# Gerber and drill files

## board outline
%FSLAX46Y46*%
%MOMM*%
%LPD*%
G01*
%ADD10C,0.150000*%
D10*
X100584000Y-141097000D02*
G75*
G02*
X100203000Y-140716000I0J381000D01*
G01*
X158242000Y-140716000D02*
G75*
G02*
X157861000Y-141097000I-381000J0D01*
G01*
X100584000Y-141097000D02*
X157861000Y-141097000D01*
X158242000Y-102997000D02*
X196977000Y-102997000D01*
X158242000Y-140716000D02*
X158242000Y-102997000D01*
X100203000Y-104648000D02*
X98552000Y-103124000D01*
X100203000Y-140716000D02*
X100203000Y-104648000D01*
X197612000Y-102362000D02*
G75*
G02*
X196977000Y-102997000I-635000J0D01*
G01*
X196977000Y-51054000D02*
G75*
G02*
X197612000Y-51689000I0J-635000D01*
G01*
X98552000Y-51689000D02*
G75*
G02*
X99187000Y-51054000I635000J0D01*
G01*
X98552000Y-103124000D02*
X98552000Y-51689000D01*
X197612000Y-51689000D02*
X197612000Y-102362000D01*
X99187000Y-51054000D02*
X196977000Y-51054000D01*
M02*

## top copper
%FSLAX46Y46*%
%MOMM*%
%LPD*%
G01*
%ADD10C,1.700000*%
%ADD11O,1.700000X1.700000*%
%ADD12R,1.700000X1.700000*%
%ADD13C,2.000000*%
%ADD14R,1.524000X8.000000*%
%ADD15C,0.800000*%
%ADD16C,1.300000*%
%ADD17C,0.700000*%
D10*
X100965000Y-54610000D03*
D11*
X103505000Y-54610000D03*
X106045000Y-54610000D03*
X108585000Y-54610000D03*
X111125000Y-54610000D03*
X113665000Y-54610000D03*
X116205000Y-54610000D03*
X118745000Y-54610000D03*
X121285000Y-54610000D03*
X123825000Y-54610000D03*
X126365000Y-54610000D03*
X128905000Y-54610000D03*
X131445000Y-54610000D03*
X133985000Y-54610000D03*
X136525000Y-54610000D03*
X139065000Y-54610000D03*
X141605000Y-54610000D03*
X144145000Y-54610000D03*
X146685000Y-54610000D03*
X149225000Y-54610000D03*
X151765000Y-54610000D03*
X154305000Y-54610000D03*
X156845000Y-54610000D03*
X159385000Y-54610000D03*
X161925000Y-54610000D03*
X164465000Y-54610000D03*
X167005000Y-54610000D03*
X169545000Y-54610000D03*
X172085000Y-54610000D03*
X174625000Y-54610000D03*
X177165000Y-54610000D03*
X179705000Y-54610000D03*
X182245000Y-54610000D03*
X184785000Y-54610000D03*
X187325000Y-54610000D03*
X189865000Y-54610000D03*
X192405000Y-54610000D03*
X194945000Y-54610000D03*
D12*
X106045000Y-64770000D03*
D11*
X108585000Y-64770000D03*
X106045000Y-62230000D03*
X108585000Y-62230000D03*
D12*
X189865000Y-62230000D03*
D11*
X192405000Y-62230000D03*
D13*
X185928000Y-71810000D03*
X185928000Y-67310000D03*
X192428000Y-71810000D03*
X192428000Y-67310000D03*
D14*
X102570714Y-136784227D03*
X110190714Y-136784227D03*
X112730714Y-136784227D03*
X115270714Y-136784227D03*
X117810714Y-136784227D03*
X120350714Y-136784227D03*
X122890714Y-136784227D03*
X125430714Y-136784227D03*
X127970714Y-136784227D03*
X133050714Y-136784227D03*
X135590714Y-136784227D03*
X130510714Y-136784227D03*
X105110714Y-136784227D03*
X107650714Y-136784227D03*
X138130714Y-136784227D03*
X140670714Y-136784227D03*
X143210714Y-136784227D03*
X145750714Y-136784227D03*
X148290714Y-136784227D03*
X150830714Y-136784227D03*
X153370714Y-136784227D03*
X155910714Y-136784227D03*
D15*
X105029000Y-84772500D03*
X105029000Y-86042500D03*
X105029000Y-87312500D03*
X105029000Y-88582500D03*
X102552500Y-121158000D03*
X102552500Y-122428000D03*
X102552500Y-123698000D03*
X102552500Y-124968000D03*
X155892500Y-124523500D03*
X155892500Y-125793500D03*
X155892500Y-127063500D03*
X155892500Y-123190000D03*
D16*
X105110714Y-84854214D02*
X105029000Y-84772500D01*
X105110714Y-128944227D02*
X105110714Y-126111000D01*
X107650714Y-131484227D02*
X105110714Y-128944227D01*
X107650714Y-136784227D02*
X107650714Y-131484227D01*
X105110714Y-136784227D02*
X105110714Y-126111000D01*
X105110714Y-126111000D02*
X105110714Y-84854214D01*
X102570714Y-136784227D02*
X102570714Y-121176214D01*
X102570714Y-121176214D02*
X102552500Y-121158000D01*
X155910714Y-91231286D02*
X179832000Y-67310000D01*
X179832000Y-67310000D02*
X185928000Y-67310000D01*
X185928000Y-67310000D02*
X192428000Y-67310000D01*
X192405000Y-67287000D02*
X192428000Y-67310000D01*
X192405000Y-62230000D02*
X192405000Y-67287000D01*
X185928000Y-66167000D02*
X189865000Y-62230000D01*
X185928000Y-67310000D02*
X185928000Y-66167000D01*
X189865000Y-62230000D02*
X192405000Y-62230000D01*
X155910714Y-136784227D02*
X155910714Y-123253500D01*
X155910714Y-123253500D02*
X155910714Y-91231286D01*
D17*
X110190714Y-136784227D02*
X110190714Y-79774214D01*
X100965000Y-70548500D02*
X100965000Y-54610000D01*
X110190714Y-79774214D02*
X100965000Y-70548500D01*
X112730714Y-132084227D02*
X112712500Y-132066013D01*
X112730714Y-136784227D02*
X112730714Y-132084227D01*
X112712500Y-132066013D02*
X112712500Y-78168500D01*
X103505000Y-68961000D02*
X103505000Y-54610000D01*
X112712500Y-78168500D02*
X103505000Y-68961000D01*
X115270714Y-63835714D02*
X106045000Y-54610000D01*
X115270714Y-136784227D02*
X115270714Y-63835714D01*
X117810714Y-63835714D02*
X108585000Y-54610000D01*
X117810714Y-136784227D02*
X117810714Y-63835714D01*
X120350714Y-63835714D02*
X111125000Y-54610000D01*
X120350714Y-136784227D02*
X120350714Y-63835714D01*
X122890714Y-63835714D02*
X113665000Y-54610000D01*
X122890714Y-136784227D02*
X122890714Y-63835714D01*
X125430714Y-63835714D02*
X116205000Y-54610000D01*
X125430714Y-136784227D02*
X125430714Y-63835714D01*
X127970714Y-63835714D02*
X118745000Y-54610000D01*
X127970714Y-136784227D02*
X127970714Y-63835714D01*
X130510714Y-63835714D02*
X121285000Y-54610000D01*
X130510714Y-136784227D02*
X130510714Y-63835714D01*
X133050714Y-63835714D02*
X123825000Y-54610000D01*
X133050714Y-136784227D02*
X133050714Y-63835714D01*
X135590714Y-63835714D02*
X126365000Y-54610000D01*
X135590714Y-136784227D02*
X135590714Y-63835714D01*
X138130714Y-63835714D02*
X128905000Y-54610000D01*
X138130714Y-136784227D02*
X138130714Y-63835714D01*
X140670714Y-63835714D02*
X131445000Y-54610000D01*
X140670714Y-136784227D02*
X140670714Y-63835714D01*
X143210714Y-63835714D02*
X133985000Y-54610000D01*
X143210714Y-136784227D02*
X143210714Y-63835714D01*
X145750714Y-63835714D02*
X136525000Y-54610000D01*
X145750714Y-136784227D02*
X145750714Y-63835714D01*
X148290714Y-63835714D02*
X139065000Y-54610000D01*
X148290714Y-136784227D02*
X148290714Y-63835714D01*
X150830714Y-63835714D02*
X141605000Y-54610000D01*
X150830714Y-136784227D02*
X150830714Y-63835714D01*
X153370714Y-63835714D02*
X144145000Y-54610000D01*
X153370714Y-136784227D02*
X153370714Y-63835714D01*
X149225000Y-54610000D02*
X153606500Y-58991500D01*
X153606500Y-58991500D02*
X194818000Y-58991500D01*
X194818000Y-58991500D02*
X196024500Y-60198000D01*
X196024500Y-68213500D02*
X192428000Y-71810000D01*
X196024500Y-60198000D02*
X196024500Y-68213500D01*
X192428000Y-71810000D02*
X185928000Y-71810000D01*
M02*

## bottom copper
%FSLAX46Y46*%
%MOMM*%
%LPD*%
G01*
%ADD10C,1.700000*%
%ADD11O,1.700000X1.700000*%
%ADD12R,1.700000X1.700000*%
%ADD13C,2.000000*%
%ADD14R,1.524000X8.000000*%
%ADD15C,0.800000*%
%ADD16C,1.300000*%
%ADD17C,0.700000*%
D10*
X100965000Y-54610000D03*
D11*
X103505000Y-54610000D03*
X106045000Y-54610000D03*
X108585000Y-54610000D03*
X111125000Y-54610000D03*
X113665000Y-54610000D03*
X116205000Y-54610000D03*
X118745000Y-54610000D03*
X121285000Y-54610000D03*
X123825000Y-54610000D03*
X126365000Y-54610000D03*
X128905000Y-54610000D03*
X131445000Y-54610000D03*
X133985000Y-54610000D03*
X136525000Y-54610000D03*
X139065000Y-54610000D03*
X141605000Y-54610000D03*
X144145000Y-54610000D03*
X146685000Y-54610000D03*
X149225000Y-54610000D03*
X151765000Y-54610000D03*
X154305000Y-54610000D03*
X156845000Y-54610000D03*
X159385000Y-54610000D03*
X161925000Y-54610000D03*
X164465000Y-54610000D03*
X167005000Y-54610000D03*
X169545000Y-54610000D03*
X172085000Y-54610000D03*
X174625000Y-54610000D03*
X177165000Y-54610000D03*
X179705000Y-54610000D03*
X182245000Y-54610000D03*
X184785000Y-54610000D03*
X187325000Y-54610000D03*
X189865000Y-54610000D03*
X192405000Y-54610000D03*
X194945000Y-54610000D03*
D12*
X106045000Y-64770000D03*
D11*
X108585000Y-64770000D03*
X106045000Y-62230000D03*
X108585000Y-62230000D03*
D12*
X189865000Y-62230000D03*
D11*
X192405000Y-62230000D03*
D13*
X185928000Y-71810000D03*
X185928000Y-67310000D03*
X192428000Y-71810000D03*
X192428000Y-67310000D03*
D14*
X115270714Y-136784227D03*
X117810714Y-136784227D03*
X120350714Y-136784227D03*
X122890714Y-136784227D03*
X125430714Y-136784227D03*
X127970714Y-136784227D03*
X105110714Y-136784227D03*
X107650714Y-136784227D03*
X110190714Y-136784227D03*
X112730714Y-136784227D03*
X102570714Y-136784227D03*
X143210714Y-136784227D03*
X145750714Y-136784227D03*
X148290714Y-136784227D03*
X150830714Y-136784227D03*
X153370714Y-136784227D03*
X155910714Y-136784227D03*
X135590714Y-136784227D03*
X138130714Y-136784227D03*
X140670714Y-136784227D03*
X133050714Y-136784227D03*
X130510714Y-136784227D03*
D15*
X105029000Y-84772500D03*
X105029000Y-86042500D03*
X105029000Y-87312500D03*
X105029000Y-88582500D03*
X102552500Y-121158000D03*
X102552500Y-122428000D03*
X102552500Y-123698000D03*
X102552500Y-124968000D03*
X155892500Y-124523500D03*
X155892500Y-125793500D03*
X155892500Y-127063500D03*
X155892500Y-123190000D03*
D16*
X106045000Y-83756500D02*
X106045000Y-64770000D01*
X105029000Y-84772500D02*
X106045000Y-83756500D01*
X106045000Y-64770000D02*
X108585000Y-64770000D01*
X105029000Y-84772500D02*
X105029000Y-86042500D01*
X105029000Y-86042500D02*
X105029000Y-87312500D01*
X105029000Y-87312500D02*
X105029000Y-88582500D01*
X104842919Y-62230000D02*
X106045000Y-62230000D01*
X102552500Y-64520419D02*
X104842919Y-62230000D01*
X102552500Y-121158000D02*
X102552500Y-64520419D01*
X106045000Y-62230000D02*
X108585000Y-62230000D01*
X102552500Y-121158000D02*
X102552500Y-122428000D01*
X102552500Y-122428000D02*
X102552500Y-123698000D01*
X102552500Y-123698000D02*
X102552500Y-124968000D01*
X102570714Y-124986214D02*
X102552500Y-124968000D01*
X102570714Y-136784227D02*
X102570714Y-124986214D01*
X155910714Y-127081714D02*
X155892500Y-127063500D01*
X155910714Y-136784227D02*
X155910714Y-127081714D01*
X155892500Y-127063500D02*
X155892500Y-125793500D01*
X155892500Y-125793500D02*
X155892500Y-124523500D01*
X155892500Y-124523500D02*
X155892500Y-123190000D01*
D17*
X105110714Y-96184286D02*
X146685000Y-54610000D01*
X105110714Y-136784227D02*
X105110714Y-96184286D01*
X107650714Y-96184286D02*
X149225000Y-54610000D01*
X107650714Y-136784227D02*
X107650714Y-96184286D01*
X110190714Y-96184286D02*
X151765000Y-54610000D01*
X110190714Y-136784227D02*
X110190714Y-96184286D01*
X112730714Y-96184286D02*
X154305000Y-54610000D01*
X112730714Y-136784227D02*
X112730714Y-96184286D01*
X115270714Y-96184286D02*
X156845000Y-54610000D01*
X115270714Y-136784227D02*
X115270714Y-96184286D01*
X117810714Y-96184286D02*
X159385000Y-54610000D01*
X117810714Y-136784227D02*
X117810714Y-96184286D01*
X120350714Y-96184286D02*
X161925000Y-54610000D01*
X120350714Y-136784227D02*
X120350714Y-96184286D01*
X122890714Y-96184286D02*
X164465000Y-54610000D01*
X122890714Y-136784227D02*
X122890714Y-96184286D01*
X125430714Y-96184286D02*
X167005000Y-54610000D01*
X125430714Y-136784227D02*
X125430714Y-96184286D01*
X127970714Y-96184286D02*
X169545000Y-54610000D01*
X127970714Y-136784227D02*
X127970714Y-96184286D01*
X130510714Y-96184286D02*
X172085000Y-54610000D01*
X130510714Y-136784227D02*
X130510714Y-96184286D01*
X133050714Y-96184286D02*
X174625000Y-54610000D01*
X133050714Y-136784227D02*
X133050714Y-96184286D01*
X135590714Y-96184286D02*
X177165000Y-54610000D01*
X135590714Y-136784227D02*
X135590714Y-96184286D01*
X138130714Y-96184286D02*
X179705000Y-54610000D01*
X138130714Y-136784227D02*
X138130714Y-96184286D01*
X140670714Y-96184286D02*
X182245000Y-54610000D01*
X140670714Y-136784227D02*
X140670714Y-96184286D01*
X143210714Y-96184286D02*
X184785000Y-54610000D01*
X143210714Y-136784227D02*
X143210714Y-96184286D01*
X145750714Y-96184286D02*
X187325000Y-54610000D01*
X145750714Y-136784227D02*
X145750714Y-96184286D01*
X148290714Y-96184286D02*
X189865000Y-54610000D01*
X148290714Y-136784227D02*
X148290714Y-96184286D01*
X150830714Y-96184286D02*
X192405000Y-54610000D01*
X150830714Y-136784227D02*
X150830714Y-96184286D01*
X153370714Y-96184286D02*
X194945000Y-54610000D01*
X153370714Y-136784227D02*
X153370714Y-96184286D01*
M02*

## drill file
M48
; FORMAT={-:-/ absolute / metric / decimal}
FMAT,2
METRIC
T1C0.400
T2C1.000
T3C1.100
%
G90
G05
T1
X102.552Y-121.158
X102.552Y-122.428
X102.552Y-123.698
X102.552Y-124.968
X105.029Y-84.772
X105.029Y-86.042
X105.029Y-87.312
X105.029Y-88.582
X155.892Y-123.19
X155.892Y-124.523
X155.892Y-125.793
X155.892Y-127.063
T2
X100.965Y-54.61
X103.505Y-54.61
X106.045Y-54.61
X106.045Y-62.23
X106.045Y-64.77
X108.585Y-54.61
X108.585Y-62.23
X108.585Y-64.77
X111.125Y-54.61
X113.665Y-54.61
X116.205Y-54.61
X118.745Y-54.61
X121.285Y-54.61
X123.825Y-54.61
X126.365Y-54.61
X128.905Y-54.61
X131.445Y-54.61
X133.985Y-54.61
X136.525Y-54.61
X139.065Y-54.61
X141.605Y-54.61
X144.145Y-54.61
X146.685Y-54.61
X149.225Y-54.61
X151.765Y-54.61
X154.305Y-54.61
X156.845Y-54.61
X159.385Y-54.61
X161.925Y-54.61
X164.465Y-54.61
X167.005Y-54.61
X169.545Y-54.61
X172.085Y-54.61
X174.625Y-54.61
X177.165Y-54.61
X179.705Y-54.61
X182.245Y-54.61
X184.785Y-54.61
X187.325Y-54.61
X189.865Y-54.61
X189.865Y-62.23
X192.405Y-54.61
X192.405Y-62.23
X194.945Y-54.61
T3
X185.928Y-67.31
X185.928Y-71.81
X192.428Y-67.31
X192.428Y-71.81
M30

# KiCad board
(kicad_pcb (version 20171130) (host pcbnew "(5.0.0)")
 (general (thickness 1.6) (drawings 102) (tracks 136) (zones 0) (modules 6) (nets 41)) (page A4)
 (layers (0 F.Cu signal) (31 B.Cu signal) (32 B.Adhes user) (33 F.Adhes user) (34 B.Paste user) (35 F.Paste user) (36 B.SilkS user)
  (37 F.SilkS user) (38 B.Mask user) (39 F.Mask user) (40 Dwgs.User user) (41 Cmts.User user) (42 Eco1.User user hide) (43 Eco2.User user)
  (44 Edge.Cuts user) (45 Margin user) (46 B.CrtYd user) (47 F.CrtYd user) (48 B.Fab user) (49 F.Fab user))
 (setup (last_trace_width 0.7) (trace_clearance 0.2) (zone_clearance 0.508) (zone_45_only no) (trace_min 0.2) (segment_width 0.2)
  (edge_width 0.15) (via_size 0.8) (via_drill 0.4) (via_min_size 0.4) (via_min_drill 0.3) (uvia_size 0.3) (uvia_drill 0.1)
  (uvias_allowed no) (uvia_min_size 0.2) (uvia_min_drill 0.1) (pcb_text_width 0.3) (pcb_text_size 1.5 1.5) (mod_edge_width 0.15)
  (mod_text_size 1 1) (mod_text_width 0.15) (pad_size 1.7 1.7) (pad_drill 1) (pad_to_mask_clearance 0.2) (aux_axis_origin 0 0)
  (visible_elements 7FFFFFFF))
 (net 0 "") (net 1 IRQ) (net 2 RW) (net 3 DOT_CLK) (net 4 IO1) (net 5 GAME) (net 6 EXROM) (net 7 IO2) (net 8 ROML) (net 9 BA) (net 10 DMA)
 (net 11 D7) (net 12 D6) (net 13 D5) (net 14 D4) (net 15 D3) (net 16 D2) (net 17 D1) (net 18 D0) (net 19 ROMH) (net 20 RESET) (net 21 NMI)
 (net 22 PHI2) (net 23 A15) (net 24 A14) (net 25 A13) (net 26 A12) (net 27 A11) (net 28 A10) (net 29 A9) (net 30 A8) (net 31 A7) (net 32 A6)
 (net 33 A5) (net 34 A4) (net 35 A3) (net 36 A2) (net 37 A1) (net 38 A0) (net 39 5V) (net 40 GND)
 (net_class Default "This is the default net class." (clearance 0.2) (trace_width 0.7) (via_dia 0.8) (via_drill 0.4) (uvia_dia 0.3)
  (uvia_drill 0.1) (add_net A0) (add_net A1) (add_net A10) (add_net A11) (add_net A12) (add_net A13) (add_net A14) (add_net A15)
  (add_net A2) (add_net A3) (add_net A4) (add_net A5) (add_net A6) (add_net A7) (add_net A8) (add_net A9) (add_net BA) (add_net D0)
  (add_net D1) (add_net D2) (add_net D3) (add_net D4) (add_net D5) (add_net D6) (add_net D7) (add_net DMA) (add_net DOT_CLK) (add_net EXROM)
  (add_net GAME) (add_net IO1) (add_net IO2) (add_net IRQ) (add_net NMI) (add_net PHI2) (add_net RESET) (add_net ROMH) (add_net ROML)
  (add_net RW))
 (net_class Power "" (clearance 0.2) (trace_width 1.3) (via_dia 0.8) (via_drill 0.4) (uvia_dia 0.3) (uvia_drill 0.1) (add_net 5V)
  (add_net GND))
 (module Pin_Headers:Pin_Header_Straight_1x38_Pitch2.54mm (layer B.Cu) (at 100.965 54.61 270)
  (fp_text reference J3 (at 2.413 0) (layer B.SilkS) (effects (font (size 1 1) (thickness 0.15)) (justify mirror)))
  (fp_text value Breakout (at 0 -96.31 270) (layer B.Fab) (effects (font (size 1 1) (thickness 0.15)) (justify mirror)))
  (pad 1 thru_hole circle (at 0 0 270) (size 1.7 1.7) (drill 1) (layers *.Cu *.Mask) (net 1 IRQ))
  (pad 2 thru_hole oval (at 0 -2.54 270) (size 1.7 1.7) (drill 1) (layers *.Cu *.Mask) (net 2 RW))
  (pad 3 thru_hole oval (at 0 -5.08 270) (size 1.7 1.7) (drill 1) (layers *.Cu *.Mask) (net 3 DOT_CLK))
  (pad 4 thru_hole oval (at 0 -7.62 270) (size 1.7 1.7) (drill 1) (layers *.Cu *.Mask) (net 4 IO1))
  (pad 5 thru_hole oval (at 0 -10.16 270) (size 1.7 1.7) (drill 1) (layers *.Cu *.Mask) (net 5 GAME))
  (pad 6 thru_hole oval (at 0 -12.7 270) (size 1.7 1.7) (drill 1) (layers *.Cu *.Mask) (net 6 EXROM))
  (pad 7 thru_hole oval (at 0 -15.24 270) (size 1.7 1.7) (drill 1) (layers *.Cu *.Mask) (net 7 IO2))
  (pad 8 thru_hole oval (at 0 -17.78 270) (size 1.7 1.7) (drill 1) (layers *.Cu *.Mask) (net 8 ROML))
  (pad 9 thru_hole oval (at 0 -20.32 270) (size 1.7 1.7) (drill 1) (layers *.Cu *.Mask) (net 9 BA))
  (pad 10 thru_hole oval (at 0 -22.86 270) (size 1.7 1.7) (drill 1) (layers *.Cu *.Mask) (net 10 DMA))
  (pad 11 thru_hole oval (at 0 -25.4 270) (size 1.7 1.7) (drill 1) (layers *.Cu *.Mask) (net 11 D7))
  (pad 12 thru_hole oval (at 0 -27.94 270) (size 1.7 1.7) (drill 1) (layers *.Cu *.Mask) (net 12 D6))
  (pad 13 thru_hole oval (at 0 -30.48 270) (size 1.7 1.7) (drill 1) (layers *.Cu *.Mask) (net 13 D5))
  (pad 14 thru_hole oval (at 0 -33.02 270) (size 1.7 1.7) (drill 1) (layers *.Cu *.Mask) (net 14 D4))
  (pad 15 thru_hole oval (at 0 -35.56 270) (size 1.7 1.7) (drill 1) (layers *.Cu *.Mask) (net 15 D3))
  (pad 16 thru_hole oval (at 0 -38.1 270) (size 1.7 1.7) (drill 1) (layers *.Cu *.Mask) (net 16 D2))
  (pad 17 thru_hole oval (at 0 -40.64 270) (size 1.7 1.7) (drill 1) (layers *.Cu *.Mask) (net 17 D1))
  (pad 18 thru_hole oval (at 0 -43.18 270) (size 1.7 1.7) (drill 1) (layers *.Cu *.Mask) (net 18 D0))
  (pad 19 thru_hole oval (at 0 -45.72 270) (size 1.7 1.7) (drill 1) (layers *.Cu *.Mask) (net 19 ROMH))
  (pad 20 thru_hole oval (at 0 -48.26 270) (size 1.7 1.7) (drill 1) (layers *.Cu *.Mask) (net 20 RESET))
  (pad 21 thru_hole oval (at 0 -50.8 270) (size 1.7 1.7) (drill 1) (layers *.Cu *.Mask) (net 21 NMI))
  (pad 22 thru_hole oval (at 0 -53.34 270) (size 1.7 1.7) (drill 1) (layers *.Cu *.Mask) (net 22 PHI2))
  (pad 23 thru_hole oval (at 0 -55.88 270) (size 1.7 1.7) (drill 1) (layers *.Cu *.Mask) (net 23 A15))
  (pad 24 thru_hole oval (at 0 -58.42 270) (size 1.7 1.7) (drill 1) (layers *.Cu *.Mask) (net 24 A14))
  (pad 25 thru_hole oval (at 0 -60.96 270) (size 1.7 1.7) (drill 1) (layers *.Cu *.Mask) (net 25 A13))
  (pad 26 thru_hole oval (at 0 -63.5 270) (size 1.7 1.7) (drill 1) (layers *.Cu *.Mask) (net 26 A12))
  (pad 27 thru_hole oval (at 0 -66.04 270) (size 1.7 1.7) (drill 1) (layers *.Cu *.Mask) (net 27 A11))
  (pad 28 thru_hole oval (at 0 -68.58 270) (size 1.7 1.7) (drill 1) (layers *.Cu *.Mask) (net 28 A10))
  (pad 29 thru_hole oval (at 0 -71.12 270) (size 1.7 1.7) (drill 1) (layers *.Cu *.Mask) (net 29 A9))
  (pad 30 thru_hole oval (at 0 -73.66 270) (size 1.7 1.7) (drill 1) (layers *.Cu *.Mask) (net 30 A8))
  (pad 31 thru_hole oval (at 0 -76.2 270) (size 1.7 1.7) (drill 1) (layers *.Cu *.Mask) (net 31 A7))
  (pad 32 thru_hole oval (at 0 -78.74 270) (size 1.7 1.7) (drill 1) (layers *.Cu *.Mask) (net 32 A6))
  (pad 33 thru_hole oval (at 0 -81.28 270) (size 1.7 1.7) (drill 1) (layers *.Cu *.Mask) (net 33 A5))
  (pad 34 thru_hole oval (at 0 -83.82 270) (size 1.7 1.7) (drill 1) (layers *.Cu *.Mask) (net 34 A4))
  (pad 35 thru_hole oval (at 0 -86.36 270) (size 1.7 1.7) (drill 1) (layers *.Cu *.Mask) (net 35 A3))
  (pad 36 thru_hole oval (at 0 -88.9 270) (size 1.7 1.7) (drill 1) (layers *.Cu *.Mask) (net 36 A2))
  (pad 37 thru_hole oval (at 0 -91.44 270) (size 1.7 1.7) (drill 1) (layers *.Cu *.Mask) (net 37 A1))
  (pad 38 thru_hole oval (at 0 -93.98 270) (size 1.7 1.7) (drill 1) (layers *.Cu *.Mask) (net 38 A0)))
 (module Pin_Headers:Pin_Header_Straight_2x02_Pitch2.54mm (layer B.Cu) (at 106.045 64.77)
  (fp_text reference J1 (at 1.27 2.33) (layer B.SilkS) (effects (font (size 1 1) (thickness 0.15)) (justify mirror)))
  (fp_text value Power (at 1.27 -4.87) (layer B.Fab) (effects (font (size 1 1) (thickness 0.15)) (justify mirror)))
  (pad 1 thru_hole rect (at 0 0) (size 1.7 1.7) (drill 1) (layers *.Cu *.Mask) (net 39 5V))
  (pad 2 thru_hole oval (at 2.54 0) (size 1.7 1.7) (drill 1) (layers *.Cu *.Mask) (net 39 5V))
  (pad 3 thru_hole oval (at 0 -2.54) (size 1.7 1.7) (drill 1) (layers *.Cu *.Mask) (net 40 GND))
  (pad 4 thru_hole oval (at 2.54 -2.54) (size 1.7 1.7) (drill 1) (layers *.Cu *.Mask) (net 40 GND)))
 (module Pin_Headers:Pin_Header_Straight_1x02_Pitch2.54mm (layer B.Cu) (at 189.865 62.23 270)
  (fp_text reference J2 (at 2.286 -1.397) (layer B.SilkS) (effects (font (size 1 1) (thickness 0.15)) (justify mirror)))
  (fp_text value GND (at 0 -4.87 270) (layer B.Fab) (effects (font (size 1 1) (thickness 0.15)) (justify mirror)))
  (pad 1 thru_hole rect (at 0 0 270) (size 1.7 1.7) (drill 1) (layers *.Cu *.Mask) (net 40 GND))
  (pad 2 thru_hole oval (at 0 -2.54 270) (size 1.7 1.7) (drill 1) (layers *.Cu *.Mask) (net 40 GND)))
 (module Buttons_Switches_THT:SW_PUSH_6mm (layer F.Cu) (at 185.928 67.31)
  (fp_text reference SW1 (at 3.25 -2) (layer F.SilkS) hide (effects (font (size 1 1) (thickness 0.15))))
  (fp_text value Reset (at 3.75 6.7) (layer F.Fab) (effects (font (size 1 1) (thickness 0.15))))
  (pad 2 thru_hole circle (at 0 4.5 90) (size 2 2) (drill 1.1) (layers *.Cu *.Mask) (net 20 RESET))
  (pad 1 thru_hole circle (at 0 0 90) (size 2 2) (drill 1.1) (layers *.Cu *.Mask) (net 40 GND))
  (pad 2 thru_hole circle (at 6.5 4.5 90) (size 2 2) (drill 1.1) (layers *.Cu *.Mask) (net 20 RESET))
  (pad 1 thru_hole circle (at 6.5 0 90) (size 2 2) (drill 1.1) (layers *.Cu *.Mask) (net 40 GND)))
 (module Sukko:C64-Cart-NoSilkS (layer F.Cu) (at 100.030714 140.722501)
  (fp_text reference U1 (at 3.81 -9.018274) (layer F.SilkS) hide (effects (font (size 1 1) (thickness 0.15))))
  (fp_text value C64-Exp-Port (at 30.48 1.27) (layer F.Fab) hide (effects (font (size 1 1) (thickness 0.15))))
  (pad 1 smd rect (at 2.54 -3.938274 180) (size 1.524 8) (layers F.Cu F.Paste F.Mask) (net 40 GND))
  (pad 4 smd rect (at 10.16 -3.938274 180) (size 1.524 8) (layers F.Cu F.Paste F.Mask) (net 1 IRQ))
  (pad 5 smd rect (at 12.7 -3.938274 180) (size 1.524 8) (layers F.Cu F.Paste F.Mask) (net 2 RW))
  (pad 6 smd rect (at 15.24 -3.938274 180) (size 1.524 8) (layers F.Cu F.Paste F.Mask) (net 3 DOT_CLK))
  (pad 7 smd rect (at 17.78 -3.938274 180) (size 1.524 8) (layers F.Cu F.Paste F.Mask) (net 4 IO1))
  (pad 8 smd rect (at 20.32 -3.938274 180) (size 1.524 8) (layers F.Cu F.Paste F.Mask) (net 5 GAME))
  (pad 9 smd rect (at 22.86 -3.938274 180) (size 1.524 8) (layers F.Cu F.Paste F.Mask) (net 6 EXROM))
  (pad 10 smd rect (at 25.4 -3.938274 180) (size 1.524 8) (layers F.Cu F.Paste F.Mask) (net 7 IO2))
  (pad 11 smd rect (at 27.94 -3.938274 180) (size 1.524 8) (layers F.Cu F.Paste F.Mask) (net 8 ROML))
  (pad 13 smd rect (at 33.02 -3.938274 180) (size 1.524 8) (layers F.Cu F.Paste F.Mask) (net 10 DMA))
  (pad 14 smd rect (at 35.56 -3.938274 180) (size 1.524 8) (layers F.Cu F.Paste F.Mask) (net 11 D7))
  (pad 12 smd rect (at 30.48 -3.938274 180) (size 1.524 8) (layers F.Cu F.Paste F.Mask) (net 9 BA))
  (pad 2 smd rect (at 5.08 -3.938274 180) (size 1.524 8) (layers F.Cu F.Paste F.Mask) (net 39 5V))
  (pad 3 smd rect (at 7.62 -3.938274 180) (size 1.524 8) (layers F.Cu F.Paste F.Mask) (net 39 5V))
  (pad 15 smd rect (at 38.1 -3.938274 180) (size 1.524 8) (layers F.Cu F.Paste F.Mask) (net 12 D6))
  (pad 16 smd rect (at 40.64 -3.938274 180) (size 1.524 8) (layers F.Cu F.Paste F.Mask) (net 13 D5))
  (pad 17 smd rect (at 43.18 -3.938274 180) (size 1.524 8) (layers F.Cu F.Paste F.Mask) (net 14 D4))
  (pad 18 smd rect (at 45.72 -3.938274 180) (size 1.524 8) (layers F.Cu F.Paste F.Mask) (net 15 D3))
  (pad 19 smd rect (at 48.26 -3.938274 180) (size 1.524 8) (layers F.Cu F.Paste F.Mask) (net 16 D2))
  (pad 20 smd rect (at 50.8 -3.938274 180) (size 1.524 8) (layers F.Cu F.Paste F.Mask) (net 17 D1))
  (pad 21 smd rect (at 53.34 -3.938274 180) (size 1.524 8) (layers F.Cu F.Paste F.Mask) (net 18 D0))
  (pad 22 smd rect (at 55.88 -3.938274 180) (size 1.524 8) (layers F.Cu F.Paste F.Mask) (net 40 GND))
  (pad F smd rect (at 15.24 -3.938274) (size 1.524 8) (layers B.Cu B.Paste B.Mask) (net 23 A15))
  (pad H smd rect (at 17.78 -3.938274) (size 1.524 8) (layers B.Cu B.Paste B.Mask) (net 24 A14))
  (pad J smd rect (at 20.32 -3.938274) (size 1.524 8) (layers B.Cu B.Paste B.Mask) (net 25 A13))
  (pad K smd rect (at 22.86 -3.938274) (size 1.524 8) (layers B.Cu B.Paste B.Mask) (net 26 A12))
  (pad L smd rect (at 25.4 -3.938274) (size 1.524 8) (layers B.Cu B.Paste B.Mask) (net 27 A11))
  (pad M smd rect (at 27.94 -3.938274) (size 1.524 8) (layers B.Cu B.Paste B.Mask) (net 28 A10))
  (pad B smd rect (at 5.08 -3.938274) (size 1.524 8) (layers B.Cu B.Paste B.Mask) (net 19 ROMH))
  (pad C smd rect (at 7.62 -3.938274) (size 1.524 8) (layers B.Cu B.Paste B.Mask) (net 20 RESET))
  (pad D smd rect (at 10.16 -3.938274) (size 1.524 8) (layers B.Cu B.Paste B.Mask) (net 21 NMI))
  (pad E smd rect (at 12.7 -3.938274) (size 1.524 8) (layers B.Cu B.Paste B.Mask) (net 22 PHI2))
  (pad A smd rect (at 2.54 -3.938274) (size 1.524 8) (layers B.Cu B.Paste B.Mask) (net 40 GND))
  (pad U smd rect (at 43.18 -3.938274) (size 1.524 8) (layers B.Cu B.Paste B.Mask) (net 34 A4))
  (pad V smd rect (at 45.72 -3.938274) (size 1.524 8) (layers B.Cu B.Paste B.Mask) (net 35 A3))
  (pad W smd rect (at 48.26 -3.938274) (size 1.524 8) (layers B.Cu B.Paste B.Mask) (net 36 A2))
  (pad X smd rect (at 50.8 -3.938274) (size 1.524 8) (layers B.Cu B.Paste B.Mask) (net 37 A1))
  (pad Y smd rect (at 53.34 -3.938274) (size 1.524 8) (layers B.Cu B.Paste B.Mask) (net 38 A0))
  (pad Z smd rect (at 55.88 -3.938274) (size 1.524 8) (layers B.Cu B.Paste B.Mask) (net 40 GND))
  (pad R smd rect (at 35.56 -3.938274) (size 1.524 8) (layers B.Cu B.Paste B.Mask) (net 31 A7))
  (pad S smd rect (at 38.1 -3.938274) (size 1.524 8) (layers B.Cu B.Paste B.Mask) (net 32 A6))
  (pad T smd rect (at 40.64 -3.938274) (size 1.524 8) (layers B.Cu B.Paste B.Mask) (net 33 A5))
  (pad P smd rect (at 33.02 -3.938274) (size 1.524 8) (layers B.Cu B.Paste B.Mask) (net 30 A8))
  (pad N smd rect (at 30.48 -3.938274) (size 1.524 8) (layers B.Cu B.Paste B.Mask) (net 29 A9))
  (pad NoSo smd rect (at 29.21 -3.81 180) (size 58.42 8.3) (layers B.Mask))
  (pad NoSo smd rect (at 29.21 -3.81 180) (size 58.42 8.3) (layers F.Mask)))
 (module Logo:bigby (layer F.Cu) (at 193.294 92.837)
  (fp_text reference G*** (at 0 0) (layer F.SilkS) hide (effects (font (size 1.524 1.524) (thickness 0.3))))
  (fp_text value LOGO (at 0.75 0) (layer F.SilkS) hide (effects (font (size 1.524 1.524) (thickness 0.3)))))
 (gr_arc (start 100.584 140.716) (end 100.584 141.097) (angle 90) (layer Edge.Cuts) (width 0.15))
 (gr_arc (start 157.861 140.716) (end 158.242 140.716) (angle 90) (layer Edge.Cuts) (width 0.15))
 (gr_line (start 100.584 141.097) (end 157.861 141.097) (angle 90) (layer Edge.Cuts) (width 0.15))
 (gr_line (start 158.242 102.997) (end 196.977 102.997) (angle 90) (layer Edge.Cuts) (width 0.15))
 (gr_line (start 158.242 140.716) (end 158.242 102.997) (angle 90) (layer Edge.Cuts) (width 0.15))
 (gr_line (start 100.203 104.648) (end 98.552 103.124) (angle 90) (layer Edge.Cuts) (width 0.15))
 (gr_line (start 100.203 140.716) (end 100.203 104.648) (angle 90) (layer Edge.Cuts) (width 0.15))
 (gr_arc (start 196.977 102.362) (end 196.977 102.997) (angle -90) (layer Edge.Cuts) (width 0.15))
 (gr_arc (start 196.977 51.689) (end 197.612 51.689) (angle -90) (layer Edge.Cuts) (width 0.15))
 (gr_arc (start 99.187 51.689) (end 99.187 51.054) (angle -90) (layer Edge.Cuts) (width 0.15))
 (gr_line (start 98.552 103.124) (end 98.552 51.689) (layer Edge.Cuts) (width 0.15))
 (gr_line (start 197.612 51.689) (end 197.612 102.362) (layer Edge.Cuts) (width 0.15))
 (gr_line (start 99.187 51.054) (end 196.977 51.054) (layer Edge.Cuts) (width 0.15))
 (via (at 105.029 84.7725) (size 0.8) (drill 0.4) (layers F.Cu B.Cu) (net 39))
 (segment (start 105.110714 84.854214) (end 105.029 84.7725) (width 1.3) (layer F.Cu) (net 39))
 (segment (start 106.045 83.7565) (end 106.045 64.77) (width 1.3) (layer B.Cu) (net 39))
 (segment (start 105.029 84.7725) (end 106.045 83.7565) (width 1.3) (layer B.Cu) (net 39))
 (segment (start 106.045 64.77) (end 108.585 64.77) (width 1.3) (layer B.Cu) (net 39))
 (via (at 105.029 86.0425) (size 0.8) (drill 0.4) (layers F.Cu B.Cu) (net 39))
 (via (at 105.029 87.3125) (size 0.8) (drill 0.4) (layers F.Cu B.Cu) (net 39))
 (via (at 105.029 88.5825) (size 0.8) (drill 0.4) (layers F.Cu B.Cu) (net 39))
 (segment (start 105.029 84.7725) (end 105.029 86.0425) (width 1.3) (layer B.Cu) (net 39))
 (segment (start 105.029 86.0425) (end 105.029 87.3125) (width 1.3) (layer B.Cu) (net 39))
 (segment (start 105.029 87.3125) (end 105.029 88.5825) (width 1.3) (layer B.Cu) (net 39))
 (segment (start 105.110714 128.944227) (end 105.110714 126.111) (width 1.3) (layer F.Cu) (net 39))
 (segment (start 107.650714 131.484227) (end 105.110714 128.944227) (width 1.3) (layer F.Cu) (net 39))
 (segment (start 107.650714 136.784227) (end 107.650714 131.484227) (width 1.3) (layer F.Cu) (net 39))
 (segment (start 105.110714 136.784227) (end 105.110714 126.111) (width 1.3) (layer F.Cu) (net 39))
 (segment (start 105.110714 126.111) (end 105.110714 84.854214) (width 1.3) (layer F.Cu) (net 39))
 (via (at 102.5525 121.158) (size 0.8) (drill 0.4) (layers F.Cu B.Cu) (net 40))
 (segment (start 102.570714 136.784227) (end 102.570714 121.176214) (width 1.3) (layer F.Cu) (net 40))
 (segment (start 102.570714 121.176214) (end 102.5525 121.158) (width 1.3) (layer F.Cu) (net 40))
 (segment (start 104.842919 62.23) (end 106.045 62.23) (width 1.3) (layer B.Cu) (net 40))
 (segment (start 102.5525 64.520419) (end 104.842919 62.23) (width 1.3) (layer B.Cu) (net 40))
 (segment (start 102.5525 121.158) (end 102.5525 64.520419) (width 1.3) (layer B.Cu) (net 40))
 (segment (start 106.045 62.23) (end 108.585 62.23) (width 1.3) (layer B.Cu) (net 40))
 (via (at 102.5525 122.428) (size 0.8) (drill 0.4) (layers F.Cu B.Cu) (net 40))
 (via (at 102.5525 123.698) (size 0.8) (drill 0.4) (layers F.Cu B.Cu) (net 40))
 (via (at 102.5525 124.968) (size 0.8) (drill 0.4) (layers F.Cu B.Cu) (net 40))
 (segment (start 102.5525 121.158) (end 102.5525 122.428) (width 1.3) (layer B.Cu) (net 40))
 (segment (start 102.5525 122.428) (end 102.5525 123.698) (width 1.3) (layer B.Cu) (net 40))
 (segment (start 102.5525 123.698) (end 102.5525 124.968) (width 1.3) (layer B.Cu) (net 40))
 (segment (start 102.570714 124.986214) (end 102.5525 124.968) (width 1.3) (layer B.Cu) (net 40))
 (segment (start 102.570714 136.784227) (end 102.570714 124.986214) (width 1.3) (layer B.Cu) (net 40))
 (segment (start 155.910714 91.231286) (end 179.832 67.31) (width 1.3) (layer F.Cu) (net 40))
 (segment (start 179.832 67.31) (end 185.928 67.31) (width 1.3) (layer F.Cu) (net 40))
 (segment (start 185.928 67.31) (end 192.428 67.31) (width 1.3) (layer F.Cu) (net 40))
 (segment (start 192.405 67.287) (end 192.428 67.31) (width 1.3) (layer F.Cu) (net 40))
 (segment (start 192.405 62.23) (end 192.405 67.287) (width 1.3) (layer F.Cu) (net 40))
 (segment (start 185.928 66.167) (end 189.865 62.23) (width 1.3) (layer F.Cu) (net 40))
 (segment (start 185.928 67.31) (end 185.928 66.167) (width 1.3) (layer F.Cu) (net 40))
 (segment (start 189.865 62.23) (end 192.405 62.23) (width 1.3) (layer F.Cu) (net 40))
 (segment (start 155.910714 136.784227) (end 155.910714 123.2535) (width 1.3) (layer F.Cu) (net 40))
 (segment (start 155.910714 123.2535) (end 155.910714 91.231286) (width 1.3) (layer F.Cu) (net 40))
 (via (at 155.8925 124.5235) (size 0.8) (drill 0.4) (layers F.Cu B.Cu) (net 40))
 (via (at 155.8925 125.7935) (size 0.8) (drill 0.4) (layers F.Cu B.Cu) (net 40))
 (via (at 155.8925 127.0635) (size 0.8) (drill 0.4) (layers F.Cu B.Cu) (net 40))
 (via (at 155.8925 123.19) (size 0.8) (drill 0.4) (layers F.Cu B.Cu) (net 40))
 (segment (start 155.910714 127.081714) (end 155.8925 127.0635) (width 1.3) (layer B.Cu) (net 40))
 (segment (start 155.910714 136.784227) (end 155.910714 127.081714) (width 1.3) (layer B.Cu) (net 40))
 (segment (start 155.8925 127.0635) (end 155.8925 125.7935) (width 1.3) (layer B.Cu) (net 40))
 (segment (start 155.8925 125.7935) (end 155.8925 124.5235) (width 1.3) (layer B.Cu) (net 40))
 (segment (start 155.8925 124.5235) (end 155.8925 123.19) (width 1.3) (layer B.Cu) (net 40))
 (segment (start 110.190714 136.784227) (end 110.190714 79.774214) (width 0.7) (layer F.Cu) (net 1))
 (segment (start 100.965 70.5485) (end 100.965 54.61) (width 0.7) (layer F.Cu) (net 1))
 (segment (start 110.190714 79.774214) (end 100.965 70.5485) (width 0.7) (layer F.Cu) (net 1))
 (segment (start 112.730714 132.084227) (end 112.7125 132.066013) (width 0.7) (layer F.Cu) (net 2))
 (segment (start 112.730714 136.784227) (end 112.730714 132.084227) (width 0.7) (layer F.Cu) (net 2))
 (segment (start 112.7125 132.066013) (end 112.7125 78.1685) (width 0.7) (layer F.Cu) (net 2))
 (segment (start 103.505 68.961) (end 103.505 54.61) (width 0.7) (layer F.Cu) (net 2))
 (segment (start 112.7125 78.1685) (end 103.505 68.961) (width 0.7) (layer F.Cu) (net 2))
 (segment (start 115.270714 63.835714) (end 106.045 54.61) (width 0.7) (layer F.Cu) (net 3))
 (segment (start 115.270714 136.784227) (end 115.270714 63.835714) (width 0.7) (layer F.Cu) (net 3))
 (segment (start 117.810714 63.835714) (end 108.585 54.61) (width 0.7) (layer F.Cu) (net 4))
 (segment (start 117.810714 136.784227) (end 117.810714 63.835714) (width 0.7) (layer F.Cu) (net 4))
 (segment (start 120.350714 63.835714) (end 111.125 54.61) (width 0.7) (layer F.Cu) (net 5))
 (segment (start 120.350714 136.784227) (end 120.350714 63.835714) (width 0.7) (layer F.Cu) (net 5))
 (segment (start 122.890714 63.835714) (end 113.665 54.61) (width 0.7) (layer F.Cu) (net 6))
 (segment (start 122.890714 136.784227) (end 122.890714 63.835714) (width 0.7) (layer F.Cu) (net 6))
 (segment (start 125.430714 63.835714) (end 116.205 54.61) (width 0.7) (layer F.Cu) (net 7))
 (segment (start 125.430714 136.784227) (end 125.430714 63.835714) (width 0.7) (layer F.Cu) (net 7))
 (segment (start 127.970714 63.835714) (end 118.745 54.61) (width 0.7) (layer F.Cu) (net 8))
 (segment (start 127.970714 136.784227) (end 127.970714 63.835714) (width 0.7) (layer F.Cu) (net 8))
 (segment (start 130.510714 63.835714) (end 121.285 54.61) (width 0.7) (layer F.Cu) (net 9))
 (segment (start 130.510714 136.784227) (end 130.510714 63.835714) (width 0.7) (layer F.Cu) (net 9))
 (segment (start 133.050714 63.835714) (end 123.825 54.61) (width 0.7) (layer F.Cu) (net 10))
 (segment (start 133.050714 136.784227) (end 133.050714 63.835714) (width 0.7) (layer F.Cu) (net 10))
 (segment (start 135.590714 63.835714) (end 126.365 54.61) (width 0.7) (layer F.Cu) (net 11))
 (segment (start 135.590714 136.784227) (end 135.590714 63.835714) (width 0.7) (layer F.Cu) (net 11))
 (segment (start 138.130714 63.835714) (end 128.905 54.61) (width 0.7) (layer F.Cu) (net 12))
 (segment (start 138.130714 136.784227) (end 138.130714 63.835714) (width 0.7) (layer F.Cu) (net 12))
 (segment (start 140.670714 63.835714) (end 131.445 54.61) (width 0.7) (layer F.Cu) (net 13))
 (segment (start 140.670714 136.784227) (end 140.670714 63.835714) (width 0.7) (layer F.Cu) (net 13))
 (segment (start 143.210714 63.835714) (end 133.985 54.61) (width 0.7) (layer F.Cu) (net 14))
 (segment (start 143.210714 136.784227) (end 143.210714 63.835714) (width 0.7) (layer F.Cu) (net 14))
 (segment (start 145.750714 63.835714) (end 136.525 54.61) (width 0.7) (layer F.Cu) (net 15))
 (segment (start 145.750714 136.784227) (end 145.750714 63.835714) (width 0.7) (layer F.Cu) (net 15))
 (segment (start 148.290714 63.835714) (end 139.065 54.61) (width 0.7) (layer F.Cu) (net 16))
 (segment (start 148.290714 136.784227) (end 148.290714 63.835714) (width 0.7) (layer F.Cu) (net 16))
 (segment (start 150.830714 63.835714) (end 141.605 54.61) (width 0.7) (layer F.Cu) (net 17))
 (segment (start 150.830714 136.784227) (end 150.830714 63.835714) (width 0.7) (layer F.Cu) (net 17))
 (segment (start 153.370714 63.835714) (end 144.145 54.61) (width 0.7) (layer F.Cu) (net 18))
 (segment (start 153.370714 136.784227) (end 153.370714 63.835714) (width 0.7) (layer F.Cu) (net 18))
 (segment (start 105.110714 96.184286) (end 146.685 54.61) (width 0.7) (layer B.Cu) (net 19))
 (segment (start 105.110714 136.784227) (end 105.110714 96.184286) (width 0.7) (layer B.Cu) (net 19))
 (segment (start 149.225 54.61) (end 153.6065 58.9915) (width 0.7) (layer F.Cu) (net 20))
 (segment (start 153.6065 58.9915) (end 194.818 58.9915) (width 0.7) (layer F.Cu) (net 20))
 (segment (start 194.818 58.9915) (end 196.0245 60.198) (width 0.7) (layer F.Cu) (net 20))
 (segment (start 196.0245 68.2135) (end 192.428 71.81) (width 0.7) (layer F.Cu) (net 20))
 (segment (start 196.0245 60.198) (end 196.0245 68.2135) (width 0.7) (layer F.Cu) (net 20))
 (segment (start 192.428 71.81) (end 185.928 71.81) (width 0.7) (layer F.Cu) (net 20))
 (segment (start 107.650714 96.184286) (end 149.225 54.61) (width 0.7) (layer B.Cu) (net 20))
 (segment (start 107.650714 136.784227) (end 107.650714 96.184286) (width 0.7) (layer B.Cu) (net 20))
 (segment (start 110.190714 96.184286) (end 151.765 54.61) (width 0.7) (layer B.Cu) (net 21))
 (segment (start 110.190714 136.784227) (end 110.190714 96.184286) (width 0.7) (layer B.Cu) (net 21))
 (segment (start 112.730714 96.184286) (end 154.305 54.61) (width 0.7) (layer B.Cu) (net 22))
 (segment (start 112.730714 136.784227) (end 112.730714 96.184286) (width 0.7) (layer B.Cu) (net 22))
 (segment (start 115.270714 96.184286) (end 156.845 54.61) (width 0.7) (layer B.Cu) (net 23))
 (segment (start 115.270714 136.784227) (end 115.270714 96.184286) (width 0.7) (layer B.Cu) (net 23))
 (segment (start 117.810714 96.184286) (end 159.385 54.61) (width 0.7) (layer B.Cu) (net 24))
 (segment (start 117.810714 136.784227) (end 117.810714 96.184286) (width 0.7) (layer B.Cu) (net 24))
 (segment (start 120.350714 96.184286) (end 161.925 54.61) (width 0.7) (layer B.Cu) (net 25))
 (segment (start 120.350714 136.784227) (end 120.350714 96.184286) (width 0.7) (layer B.Cu) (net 25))
 (segment (start 122.890714 96.184286) (end 164.465 54.61) (width 0.7) (layer B.Cu) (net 26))
 (segment (start 122.890714 136.784227) (end 122.890714 96.184286) (width 0.7) (layer B.Cu) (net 26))
 (segment (start 125.430714 96.184286) (end 167.005 54.61) (width 0.7) (layer B.Cu) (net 27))
 (segment (start 125.430714 136.784227) (end 125.430714 96.184286) (width 0.7) (layer B.Cu) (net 27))
 (segment (start 127.970714 96.184286) (end 169.545 54.61) (width 0.7) (layer B.Cu) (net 28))
 (segment (start 127.970714 136.784227) (end 127.970714 96.184286) (width 0.7) (layer B.Cu) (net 28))
 (segment (start 130.510714 96.184286) (end 172.085 54.61) (width 0.7) (layer B.Cu) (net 29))
 (segment (start 130.510714 136.784227) (end 130.510714 96.184286) (width 0.7) (layer B.Cu) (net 29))
 (segment (start 133.050714 96.184286) (end 174.625 54.61) (width 0.7) (layer B.Cu) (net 30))
 (segment (start 133.050714 136.784227) (end 133.050714 96.184286) (width 0.7) (layer B.Cu) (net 30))
 (segment (start 135.590714 96.184286) (end 177.165 54.61) (width 0.7) (layer B.Cu) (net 31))
 (segment (start 135.590714 136.784227) (end 135.590714 96.184286) (width 0.7) (layer B.Cu) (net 31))
 (segment (start 138.130714 96.184286) (end 179.705 54.61) (width 0.7) (layer B.Cu) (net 32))
 (segment (start 138.130714 136.784227) (end 138.130714 96.184286) (width 0.7) (layer B.Cu) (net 32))
 (segment (start 140.670714 96.184286) (end 182.245 54.61) (width 0.7) (layer B.Cu) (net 33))
 (segment (start 140.670714 136.784227) (end 140.670714 96.184286) (width 0.7) (layer B.Cu) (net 33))
 (segment (start 143.210714 96.184286) (end 184.785 54.61) (width 0.7) (layer B.Cu) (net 34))
 (segment (start 143.210714 136.784227) (end 143.210714 96.184286) (width 0.7) (layer B.Cu) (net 34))
 (segment (start 145.750714 96.184286) (end 187.325 54.61) (width 0.7) (layer B.Cu) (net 35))
 (segment (start 145.750714 136.784227) (end 145.750714 96.184286) (width 0.7) (layer B.Cu) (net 35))
 (segment (start 148.290714 96.184286) (end 189.865 54.61) (width 0.7) (layer B.Cu) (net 36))
 (segment (start 148.290714 136.784227) (end 148.290714 96.184286) (width 0.7) (layer B.Cu) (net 36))
 (segment (start 150.830714 96.184286) (end 192.405 54.61) (width 0.7) (layer B.Cu) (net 37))
 (segment (start 150.830714 136.784227) (end 150.830714 96.184286) (width 0.7) (layer B.Cu) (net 37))
 (segment (start 153.370714 96.184286) (end 194.945 54.61) (width 0.7) (layer B.Cu) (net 38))
 (segment (start 153.370714 136.784227) (end 153.370714 96.184286) (width 0.7) (layer B.Cu) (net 38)))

